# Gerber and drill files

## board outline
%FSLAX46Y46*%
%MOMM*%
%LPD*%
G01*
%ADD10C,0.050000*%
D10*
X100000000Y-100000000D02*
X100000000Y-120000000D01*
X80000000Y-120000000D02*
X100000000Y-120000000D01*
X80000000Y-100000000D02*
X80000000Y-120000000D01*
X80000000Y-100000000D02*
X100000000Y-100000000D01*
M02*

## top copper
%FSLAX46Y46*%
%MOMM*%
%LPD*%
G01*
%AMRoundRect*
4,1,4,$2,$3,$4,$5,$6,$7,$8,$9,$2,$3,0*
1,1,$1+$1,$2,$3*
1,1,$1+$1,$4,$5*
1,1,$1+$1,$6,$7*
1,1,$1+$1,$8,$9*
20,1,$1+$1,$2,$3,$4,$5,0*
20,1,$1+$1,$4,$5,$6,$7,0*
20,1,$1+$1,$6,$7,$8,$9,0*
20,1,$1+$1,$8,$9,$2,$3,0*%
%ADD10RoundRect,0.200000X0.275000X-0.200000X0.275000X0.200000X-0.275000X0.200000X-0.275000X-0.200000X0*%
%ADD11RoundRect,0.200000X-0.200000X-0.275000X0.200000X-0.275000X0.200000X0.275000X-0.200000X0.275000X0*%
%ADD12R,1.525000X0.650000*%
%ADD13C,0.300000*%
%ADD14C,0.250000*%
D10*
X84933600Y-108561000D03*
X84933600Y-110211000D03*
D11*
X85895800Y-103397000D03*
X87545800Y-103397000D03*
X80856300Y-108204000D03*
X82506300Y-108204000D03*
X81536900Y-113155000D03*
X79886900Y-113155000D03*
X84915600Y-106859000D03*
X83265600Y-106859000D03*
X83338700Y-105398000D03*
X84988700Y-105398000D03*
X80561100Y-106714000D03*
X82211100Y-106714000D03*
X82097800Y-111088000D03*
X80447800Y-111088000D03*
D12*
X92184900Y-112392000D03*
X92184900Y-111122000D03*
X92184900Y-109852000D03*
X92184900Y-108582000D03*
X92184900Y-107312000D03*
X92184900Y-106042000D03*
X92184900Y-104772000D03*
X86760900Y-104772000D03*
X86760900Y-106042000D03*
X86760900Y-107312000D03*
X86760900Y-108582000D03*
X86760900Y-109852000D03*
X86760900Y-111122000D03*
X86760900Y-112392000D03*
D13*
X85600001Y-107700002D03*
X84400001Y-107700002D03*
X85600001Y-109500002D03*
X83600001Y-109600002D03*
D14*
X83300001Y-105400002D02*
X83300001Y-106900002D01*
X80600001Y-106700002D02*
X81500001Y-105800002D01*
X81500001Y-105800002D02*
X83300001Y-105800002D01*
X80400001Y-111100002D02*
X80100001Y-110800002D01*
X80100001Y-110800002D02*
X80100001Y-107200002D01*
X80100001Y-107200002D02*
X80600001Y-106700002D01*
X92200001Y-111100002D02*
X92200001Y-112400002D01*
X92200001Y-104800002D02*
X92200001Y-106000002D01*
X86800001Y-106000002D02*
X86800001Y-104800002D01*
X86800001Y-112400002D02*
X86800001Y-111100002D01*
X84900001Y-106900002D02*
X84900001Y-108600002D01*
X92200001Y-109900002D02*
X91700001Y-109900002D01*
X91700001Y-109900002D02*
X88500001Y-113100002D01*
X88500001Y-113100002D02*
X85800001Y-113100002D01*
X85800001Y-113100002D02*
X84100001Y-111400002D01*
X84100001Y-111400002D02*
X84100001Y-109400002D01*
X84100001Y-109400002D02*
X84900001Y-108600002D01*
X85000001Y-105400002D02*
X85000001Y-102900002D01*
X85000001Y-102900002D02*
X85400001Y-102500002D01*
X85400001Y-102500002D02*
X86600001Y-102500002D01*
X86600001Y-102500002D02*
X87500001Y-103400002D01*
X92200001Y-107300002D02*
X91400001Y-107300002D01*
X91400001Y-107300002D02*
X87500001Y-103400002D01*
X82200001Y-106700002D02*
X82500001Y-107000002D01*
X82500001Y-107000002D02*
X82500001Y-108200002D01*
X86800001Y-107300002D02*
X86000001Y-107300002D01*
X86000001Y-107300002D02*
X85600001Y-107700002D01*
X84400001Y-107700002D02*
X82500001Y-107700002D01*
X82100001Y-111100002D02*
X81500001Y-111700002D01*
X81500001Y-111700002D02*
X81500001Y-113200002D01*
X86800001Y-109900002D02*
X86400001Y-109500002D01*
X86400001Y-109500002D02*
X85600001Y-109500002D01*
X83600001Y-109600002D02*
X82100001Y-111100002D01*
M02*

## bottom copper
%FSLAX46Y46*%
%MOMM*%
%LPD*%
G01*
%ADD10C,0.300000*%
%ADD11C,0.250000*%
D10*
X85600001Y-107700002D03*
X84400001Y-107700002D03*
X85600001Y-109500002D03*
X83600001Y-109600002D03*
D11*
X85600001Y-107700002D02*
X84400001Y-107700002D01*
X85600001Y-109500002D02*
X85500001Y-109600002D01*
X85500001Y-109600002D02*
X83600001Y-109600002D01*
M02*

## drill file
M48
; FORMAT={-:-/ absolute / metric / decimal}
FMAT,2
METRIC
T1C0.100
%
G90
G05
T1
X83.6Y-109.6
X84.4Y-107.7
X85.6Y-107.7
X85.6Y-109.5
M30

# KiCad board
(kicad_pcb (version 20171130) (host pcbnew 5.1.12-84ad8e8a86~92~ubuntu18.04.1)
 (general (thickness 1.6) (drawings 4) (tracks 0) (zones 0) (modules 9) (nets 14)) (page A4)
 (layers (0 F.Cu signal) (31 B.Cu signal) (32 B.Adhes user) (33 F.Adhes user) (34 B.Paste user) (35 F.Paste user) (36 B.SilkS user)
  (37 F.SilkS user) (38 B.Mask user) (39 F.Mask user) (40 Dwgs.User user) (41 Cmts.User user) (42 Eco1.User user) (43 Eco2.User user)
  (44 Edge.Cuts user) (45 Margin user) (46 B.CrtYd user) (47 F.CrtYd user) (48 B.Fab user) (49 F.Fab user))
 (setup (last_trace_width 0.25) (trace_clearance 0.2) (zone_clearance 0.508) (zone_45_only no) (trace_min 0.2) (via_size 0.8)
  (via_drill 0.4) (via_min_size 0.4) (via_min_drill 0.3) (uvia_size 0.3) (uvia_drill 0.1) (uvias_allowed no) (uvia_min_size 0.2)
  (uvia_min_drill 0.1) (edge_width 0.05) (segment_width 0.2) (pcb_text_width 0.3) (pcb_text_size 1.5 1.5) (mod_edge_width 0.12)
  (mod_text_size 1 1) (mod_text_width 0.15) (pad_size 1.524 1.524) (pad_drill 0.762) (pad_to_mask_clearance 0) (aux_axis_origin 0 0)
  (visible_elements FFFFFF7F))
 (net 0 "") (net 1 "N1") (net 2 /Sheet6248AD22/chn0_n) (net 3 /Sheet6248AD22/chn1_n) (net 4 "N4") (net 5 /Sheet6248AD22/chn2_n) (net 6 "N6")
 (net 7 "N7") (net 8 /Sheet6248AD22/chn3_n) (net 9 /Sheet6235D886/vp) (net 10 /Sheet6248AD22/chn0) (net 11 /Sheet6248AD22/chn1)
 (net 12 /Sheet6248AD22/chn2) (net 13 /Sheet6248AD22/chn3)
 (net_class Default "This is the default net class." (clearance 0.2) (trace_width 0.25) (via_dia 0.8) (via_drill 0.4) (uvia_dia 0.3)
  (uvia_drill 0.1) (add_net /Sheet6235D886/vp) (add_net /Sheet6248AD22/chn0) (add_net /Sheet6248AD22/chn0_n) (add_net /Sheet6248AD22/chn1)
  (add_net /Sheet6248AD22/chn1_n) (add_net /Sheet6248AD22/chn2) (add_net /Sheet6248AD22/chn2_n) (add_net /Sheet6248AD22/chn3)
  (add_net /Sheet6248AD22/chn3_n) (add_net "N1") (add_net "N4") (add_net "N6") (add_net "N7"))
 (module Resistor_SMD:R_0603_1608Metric (layer F.Cu) (at 84.933600 109.386000 90.000000)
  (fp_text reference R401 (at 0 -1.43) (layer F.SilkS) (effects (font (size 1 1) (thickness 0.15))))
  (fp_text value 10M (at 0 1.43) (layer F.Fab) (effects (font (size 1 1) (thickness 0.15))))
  (pad 2 smd roundrect (at 0.825 0 90.000000) (size 0.8 0.95) (layers F.Cu F.Mask F.Paste) (roundrect_rratio 0.25) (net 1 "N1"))
  (pad 1 smd roundrect (at -0.825 0 90.000000) (size 0.8 0.95) (layers F.Cu F.Mask F.Paste) (roundrect_rratio 0.25)
   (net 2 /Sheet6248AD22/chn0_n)))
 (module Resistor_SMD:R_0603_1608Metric (layer F.Cu) (at 86.720800 103.397000)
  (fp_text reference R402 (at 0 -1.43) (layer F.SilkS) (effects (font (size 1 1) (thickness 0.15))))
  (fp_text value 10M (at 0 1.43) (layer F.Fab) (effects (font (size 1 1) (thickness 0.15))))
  (pad 1 smd roundrect (at -0.825 0) (size 0.8 0.95) (layers F.Cu F.Mask F.Paste) (roundrect_rratio 0.25) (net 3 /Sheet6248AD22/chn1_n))
  (pad 2 smd roundrect (at 0.825 0) (size 0.8 0.95) (layers F.Cu F.Mask F.Paste) (roundrect_rratio 0.25) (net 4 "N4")))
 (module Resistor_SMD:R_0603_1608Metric (layer F.Cu) (at 81.681300 108.204000)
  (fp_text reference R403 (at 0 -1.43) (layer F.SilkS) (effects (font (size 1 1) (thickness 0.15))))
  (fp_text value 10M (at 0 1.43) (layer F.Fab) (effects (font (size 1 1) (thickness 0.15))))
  (pad 1 smd roundrect (at -0.825 0) (size 0.8 0.95) (layers F.Cu F.Mask F.Paste) (roundrect_rratio 0.25) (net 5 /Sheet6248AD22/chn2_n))
  (pad 2 smd roundrect (at 0.825 0) (size 0.8 0.95) (layers F.Cu F.Mask F.Paste) (roundrect_rratio 0.25) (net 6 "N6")))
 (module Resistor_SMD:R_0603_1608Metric (layer F.Cu) (at 80.711900 113.155000)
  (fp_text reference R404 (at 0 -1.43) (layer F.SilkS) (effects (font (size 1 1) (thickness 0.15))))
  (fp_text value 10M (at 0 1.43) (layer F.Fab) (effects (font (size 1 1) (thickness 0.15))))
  (pad 2 smd roundrect (at 0.825 0) (size 0.8 0.95) (layers F.Cu F.Mask F.Paste) (roundrect_rratio 0.25) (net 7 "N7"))
  (pad 1 smd roundrect (at -0.825 0) (size 0.8 0.95) (layers F.Cu F.Mask F.Paste) (roundrect_rratio 0.25) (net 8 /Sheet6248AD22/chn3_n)))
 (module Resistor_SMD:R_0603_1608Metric (layer F.Cu) (at 84.090600 106.859000)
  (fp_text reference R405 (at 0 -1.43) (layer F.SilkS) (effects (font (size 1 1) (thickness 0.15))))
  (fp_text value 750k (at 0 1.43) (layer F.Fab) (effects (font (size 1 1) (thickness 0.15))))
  (pad 2 smd roundrect (at 0.825 0) (size 0.8 0.95) (layers F.Cu F.Mask F.Paste) (roundrect_rratio 0.25) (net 1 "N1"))
  (pad 1 smd roundrect (at -0.825 0) (size 0.8 0.95) (layers F.Cu F.Mask F.Paste) (roundrect_rratio 0.25) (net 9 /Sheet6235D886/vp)))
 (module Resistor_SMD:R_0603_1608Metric (layer F.Cu) (at 84.163700 105.398000)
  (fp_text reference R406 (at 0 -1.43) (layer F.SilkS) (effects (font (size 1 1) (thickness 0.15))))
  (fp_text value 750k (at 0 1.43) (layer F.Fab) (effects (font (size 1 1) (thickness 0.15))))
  (pad 1 smd roundrect (at -0.825 0) (size 0.8 0.95) (layers F.Cu F.Mask F.Paste) (roundrect_rratio 0.25) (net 9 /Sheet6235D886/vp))
  (pad 2 smd roundrect (at 0.825 0) (size 0.8 0.95) (layers F.Cu F.Mask F.Paste) (roundrect_rratio 0.25) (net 4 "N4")))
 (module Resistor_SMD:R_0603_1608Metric (layer F.Cu) (at 81.386100 106.714000)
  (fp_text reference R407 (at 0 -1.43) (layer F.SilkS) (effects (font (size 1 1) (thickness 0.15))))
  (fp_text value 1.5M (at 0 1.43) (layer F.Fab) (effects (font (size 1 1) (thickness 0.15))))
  (pad 1 smd roundrect (at -0.825 0) (size 0.8 0.95) (layers F.Cu F.Mask F.Paste) (roundrect_rratio 0.25) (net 9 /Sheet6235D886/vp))
  (pad 2 smd roundrect (at 0.825 0) (size 0.8 0.95) (layers F.Cu F.Mask F.Paste) (roundrect_rratio 0.25) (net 6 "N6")))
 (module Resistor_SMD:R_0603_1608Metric (layer F.Cu) (at 81.272800 111.088000)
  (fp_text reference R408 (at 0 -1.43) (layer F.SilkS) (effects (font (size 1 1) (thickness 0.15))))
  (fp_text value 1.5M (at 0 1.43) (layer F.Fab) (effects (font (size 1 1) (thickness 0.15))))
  (pad 2 smd roundrect (at 0.825 0) (size 0.8 0.95) (layers F.Cu F.Mask F.Paste) (roundrect_rratio 0.25) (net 7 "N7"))
  (pad 1 smd roundrect (at -0.825 0) (size 0.8 0.95) (layers F.Cu F.Mask F.Paste) (roundrect_rratio 0.25) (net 9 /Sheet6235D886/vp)))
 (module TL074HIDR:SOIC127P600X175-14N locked (layer F.Cu) (at 89.472900 108.582000 180.000000)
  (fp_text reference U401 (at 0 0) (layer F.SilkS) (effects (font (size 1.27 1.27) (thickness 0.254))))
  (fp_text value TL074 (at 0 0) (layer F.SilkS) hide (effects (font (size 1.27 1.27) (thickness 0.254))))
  (pad 1 smd rect (at -2.712 -3.81 270.000000) (size 0.65 1.525) (layers F.Cu F.Mask F.Paste) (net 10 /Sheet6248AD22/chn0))
  (pad 2 smd rect (at -2.712 -2.54 270.000000) (size 0.65 1.525) (layers F.Cu F.Mask F.Paste) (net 10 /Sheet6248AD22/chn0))
  (pad 3 smd rect (at -2.712 -1.27 270.000000) (size 0.65 1.525) (layers F.Cu F.Mask F.Paste) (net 1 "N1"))
  (pad 4 smd rect (at -2.712 0 270.000000) (size 0.65 1.525) (layers F.Cu F.Mask F.Paste))
  (pad 5 smd rect (at -2.712 1.27 270.000000) (size 0.65 1.525) (layers F.Cu F.Mask F.Paste) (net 4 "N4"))
  (pad 6 smd rect (at -2.712 2.54 270.000000) (size 0.65 1.525) (layers F.Cu F.Mask F.Paste) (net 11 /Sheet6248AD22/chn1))
  (pad 7 smd rect (at -2.712 3.81 270.000000) (size 0.65 1.525) (layers F.Cu F.Mask F.Paste) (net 11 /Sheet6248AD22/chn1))
  (pad 8 smd rect (at 2.712 3.81 270.000000) (size 0.65 1.525) (layers F.Cu F.Mask F.Paste) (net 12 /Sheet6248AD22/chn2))
  (pad 9 smd rect (at 2.712 2.54 270.000000) (size 0.65 1.525) (layers F.Cu F.Mask F.Paste) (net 12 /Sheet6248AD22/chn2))
  (pad 10 smd rect (at 2.712 1.27 270.000000) (size 0.65 1.525) (layers F.Cu F.Mask F.Paste) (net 6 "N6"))
  (pad 11 smd rect (at 2.712 0 270.000000) (size 0.65 1.525) (layers F.Cu F.Mask F.Paste))
  (pad 12 smd rect (at 2.712 -1.27 270.000000) (size 0.65 1.525) (layers F.Cu F.Mask F.Paste) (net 7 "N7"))
  (pad 13 smd rect (at 2.712 -2.54 270.000000) (size 0.65 1.525) (layers F.Cu F.Mask F.Paste) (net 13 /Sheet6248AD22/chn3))
  (pad 14 smd rect (at 2.712 -3.81 270.000000) (size 0.65 1.525) (layers F.Cu F.Mask F.Paste) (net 13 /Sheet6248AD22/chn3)))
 (gr_line (start 100 100) (end 100 120) (layer Edge.Cuts) (width 0.05))
 (gr_line (start 80 120) (end 100 120) (layer Edge.Cuts) (width 0.05))
 (gr_line (start 80 100) (end 80 120) (layer Edge.Cuts) (width 0.05))
 (gr_line (start 80 100) (end 100 100) (layer Edge.Cuts) (width 0.05))
 (segment (start 83.300001 105.400002) (end 83.300001 106.900002) (width 0.250000) (layer F.Cu) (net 9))
 (segment (start 80.600001 106.700002) (end 81.500001 105.800002) (width 0.250000) (layer F.Cu) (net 9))
 (segment (start 81.500001 105.800002) (end 83.300001 105.800002) (width 0.250000) (layer F.Cu) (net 9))
 (segment (start 80.400001 111.100002) (end 80.100001 110.800002) (width 0.250000) (layer F.Cu) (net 9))
 (segment (start 80.100001 110.800002) (end 80.100001 107.200002) (width 0.250000) (layer F.Cu) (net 9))
 (segment (start 80.100001 107.200002) (end 80.600001 106.700002) (width 0.250000) (layer F.Cu) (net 9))
 (segment (start 92.200001 111.100002) (end 92.200001 112.400002) (width 0.250000) (layer F.Cu) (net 10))
 (segment (start 92.200001 104.800002) (end 92.200001 106.000002) (width 0.250000) (layer F.Cu) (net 11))
 (segment (start 86.800001 106.000002) (end 86.800001 104.800002) (width 0.250000) (layer F.Cu) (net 12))
 (segment (start 86.800001 112.400002) (end 86.800001 111.100002) (width 0.250000) (layer F.Cu) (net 13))
 (segment (start 84.900001 106.900002) (end 84.900001 108.600002) (width 0.250000) (layer F.Cu) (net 1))
 (segment (start 92.200001 109.900002) (end 91.700001 109.900002) (width 0.250000) (layer F.Cu) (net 1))
 (segment (start 91.700001 109.900002) (end 88.500001 113.100002) (width 0.250000) (layer F.Cu) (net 1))
 (segment (start 88.500001 113.100002) (end 85.800001 113.100002) (width 0.250000) (layer F.Cu) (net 1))
 (segment (start 85.800001 113.100002) (end 84.100001 111.400002) (width 0.250000) (layer F.Cu) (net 1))
 (segment (start 84.100001 111.400002) (end 84.100001 109.400002) (width 0.250000) (layer F.Cu) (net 1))
 (segment (start 84.100001 109.400002) (end 84.900001 108.600002) (width 0.250000) (layer F.Cu) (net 1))
 (segment (start 85.000001 105.400002) (end 85.000001 102.900002) (width 0.250000) (layer F.Cu) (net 4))
 (segment (start 85.000001 102.900002) (end 85.400001 102.500002) (width 0.250000) (layer F.Cu) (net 4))
 (segment (start 85.400001 102.500002) (end 86.600001 102.500002) (width 0.250000) (layer F.Cu) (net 4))
 (segment (start 86.600001 102.500002) (end 87.500001 103.400002) (width 0.250000) (layer F.Cu) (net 4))
 (segment (start 92.200001 107.300002) (end 91.400001 107.300002) (width 0.250000) (layer F.Cu) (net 4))
 (segment (start 91.400001 107.300002) (end 87.500001 103.400002) (width 0.250000) (layer F.Cu) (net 4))
 (segment (start 82.200001 106.700002) (end 82.500001 107.000002) (width 0.250000) (layer F.Cu) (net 6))
 (segment (start 82.500001 107.000002) (end 82.500001 108.200002) (width 0.250000) (layer F.Cu) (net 6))
 (segment (start 86.800001 107.300002) (end 86.000001 107.300002) (width 0.250000) (layer F.Cu) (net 6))
 (segment (start 86.000001 107.300002) (end 85.600001 107.700002) (width 0.250000) (layer F.Cu) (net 6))
 (segment (start 85.600001 107.700002) (end 84.400001 107.700002) (width 0.250000) (layer B.Cu) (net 6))
 (segment (start 84.400001 107.700002) (end 82.500001 107.700002) (width 0.250000) (layer F.Cu) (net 6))
 (via micro (at 85.600001 107.700002) (size 0.300000) (drill 0.100000) (layers F.Cu B.Cu) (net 6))
 (via micro (at 84.400001 107.700002) (size 0.300000) (drill 0.100000) (layers F.Cu B.Cu) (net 6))
 (segment (start 82.100001 111.100002) (end 81.500001 111.700002) (width 0.250000) (layer F.Cu) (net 7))
 (segment (start 81.500001 111.700002) (end 81.500001 113.200002) (width 0.250000) (layer F.Cu) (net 7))
 (segment (start 86.800001 109.900002) (end 86.400001 109.500002) (width 0.250000) (layer F.Cu) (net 7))
 (segment (start 86.400001 109.500002) (end 85.600001 109.500002) (width 0.250000) (layer F.Cu) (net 7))
 (segment (start 85.600001 109.500002) (end 85.500001 109.600002) (width 0.250000) (layer B.Cu) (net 7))
 (segment (start 85.500001 109.600002) (end 83.600001 109.600002) (width 0.250000) (layer B.Cu) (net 7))
 (segment (start 83.600001 109.600002) (end 82.100001 111.100002) (width 0.250000) (layer F.Cu) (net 7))
 (via micro (at 85.600001 109.500002) (size 0.300000) (drill 0.100000) (layers F.Cu B.Cu) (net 7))
 (via micro (at 83.600001 109.600002) (size 0.300000) (drill 0.100000) (layers F.Cu B.Cu) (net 7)))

